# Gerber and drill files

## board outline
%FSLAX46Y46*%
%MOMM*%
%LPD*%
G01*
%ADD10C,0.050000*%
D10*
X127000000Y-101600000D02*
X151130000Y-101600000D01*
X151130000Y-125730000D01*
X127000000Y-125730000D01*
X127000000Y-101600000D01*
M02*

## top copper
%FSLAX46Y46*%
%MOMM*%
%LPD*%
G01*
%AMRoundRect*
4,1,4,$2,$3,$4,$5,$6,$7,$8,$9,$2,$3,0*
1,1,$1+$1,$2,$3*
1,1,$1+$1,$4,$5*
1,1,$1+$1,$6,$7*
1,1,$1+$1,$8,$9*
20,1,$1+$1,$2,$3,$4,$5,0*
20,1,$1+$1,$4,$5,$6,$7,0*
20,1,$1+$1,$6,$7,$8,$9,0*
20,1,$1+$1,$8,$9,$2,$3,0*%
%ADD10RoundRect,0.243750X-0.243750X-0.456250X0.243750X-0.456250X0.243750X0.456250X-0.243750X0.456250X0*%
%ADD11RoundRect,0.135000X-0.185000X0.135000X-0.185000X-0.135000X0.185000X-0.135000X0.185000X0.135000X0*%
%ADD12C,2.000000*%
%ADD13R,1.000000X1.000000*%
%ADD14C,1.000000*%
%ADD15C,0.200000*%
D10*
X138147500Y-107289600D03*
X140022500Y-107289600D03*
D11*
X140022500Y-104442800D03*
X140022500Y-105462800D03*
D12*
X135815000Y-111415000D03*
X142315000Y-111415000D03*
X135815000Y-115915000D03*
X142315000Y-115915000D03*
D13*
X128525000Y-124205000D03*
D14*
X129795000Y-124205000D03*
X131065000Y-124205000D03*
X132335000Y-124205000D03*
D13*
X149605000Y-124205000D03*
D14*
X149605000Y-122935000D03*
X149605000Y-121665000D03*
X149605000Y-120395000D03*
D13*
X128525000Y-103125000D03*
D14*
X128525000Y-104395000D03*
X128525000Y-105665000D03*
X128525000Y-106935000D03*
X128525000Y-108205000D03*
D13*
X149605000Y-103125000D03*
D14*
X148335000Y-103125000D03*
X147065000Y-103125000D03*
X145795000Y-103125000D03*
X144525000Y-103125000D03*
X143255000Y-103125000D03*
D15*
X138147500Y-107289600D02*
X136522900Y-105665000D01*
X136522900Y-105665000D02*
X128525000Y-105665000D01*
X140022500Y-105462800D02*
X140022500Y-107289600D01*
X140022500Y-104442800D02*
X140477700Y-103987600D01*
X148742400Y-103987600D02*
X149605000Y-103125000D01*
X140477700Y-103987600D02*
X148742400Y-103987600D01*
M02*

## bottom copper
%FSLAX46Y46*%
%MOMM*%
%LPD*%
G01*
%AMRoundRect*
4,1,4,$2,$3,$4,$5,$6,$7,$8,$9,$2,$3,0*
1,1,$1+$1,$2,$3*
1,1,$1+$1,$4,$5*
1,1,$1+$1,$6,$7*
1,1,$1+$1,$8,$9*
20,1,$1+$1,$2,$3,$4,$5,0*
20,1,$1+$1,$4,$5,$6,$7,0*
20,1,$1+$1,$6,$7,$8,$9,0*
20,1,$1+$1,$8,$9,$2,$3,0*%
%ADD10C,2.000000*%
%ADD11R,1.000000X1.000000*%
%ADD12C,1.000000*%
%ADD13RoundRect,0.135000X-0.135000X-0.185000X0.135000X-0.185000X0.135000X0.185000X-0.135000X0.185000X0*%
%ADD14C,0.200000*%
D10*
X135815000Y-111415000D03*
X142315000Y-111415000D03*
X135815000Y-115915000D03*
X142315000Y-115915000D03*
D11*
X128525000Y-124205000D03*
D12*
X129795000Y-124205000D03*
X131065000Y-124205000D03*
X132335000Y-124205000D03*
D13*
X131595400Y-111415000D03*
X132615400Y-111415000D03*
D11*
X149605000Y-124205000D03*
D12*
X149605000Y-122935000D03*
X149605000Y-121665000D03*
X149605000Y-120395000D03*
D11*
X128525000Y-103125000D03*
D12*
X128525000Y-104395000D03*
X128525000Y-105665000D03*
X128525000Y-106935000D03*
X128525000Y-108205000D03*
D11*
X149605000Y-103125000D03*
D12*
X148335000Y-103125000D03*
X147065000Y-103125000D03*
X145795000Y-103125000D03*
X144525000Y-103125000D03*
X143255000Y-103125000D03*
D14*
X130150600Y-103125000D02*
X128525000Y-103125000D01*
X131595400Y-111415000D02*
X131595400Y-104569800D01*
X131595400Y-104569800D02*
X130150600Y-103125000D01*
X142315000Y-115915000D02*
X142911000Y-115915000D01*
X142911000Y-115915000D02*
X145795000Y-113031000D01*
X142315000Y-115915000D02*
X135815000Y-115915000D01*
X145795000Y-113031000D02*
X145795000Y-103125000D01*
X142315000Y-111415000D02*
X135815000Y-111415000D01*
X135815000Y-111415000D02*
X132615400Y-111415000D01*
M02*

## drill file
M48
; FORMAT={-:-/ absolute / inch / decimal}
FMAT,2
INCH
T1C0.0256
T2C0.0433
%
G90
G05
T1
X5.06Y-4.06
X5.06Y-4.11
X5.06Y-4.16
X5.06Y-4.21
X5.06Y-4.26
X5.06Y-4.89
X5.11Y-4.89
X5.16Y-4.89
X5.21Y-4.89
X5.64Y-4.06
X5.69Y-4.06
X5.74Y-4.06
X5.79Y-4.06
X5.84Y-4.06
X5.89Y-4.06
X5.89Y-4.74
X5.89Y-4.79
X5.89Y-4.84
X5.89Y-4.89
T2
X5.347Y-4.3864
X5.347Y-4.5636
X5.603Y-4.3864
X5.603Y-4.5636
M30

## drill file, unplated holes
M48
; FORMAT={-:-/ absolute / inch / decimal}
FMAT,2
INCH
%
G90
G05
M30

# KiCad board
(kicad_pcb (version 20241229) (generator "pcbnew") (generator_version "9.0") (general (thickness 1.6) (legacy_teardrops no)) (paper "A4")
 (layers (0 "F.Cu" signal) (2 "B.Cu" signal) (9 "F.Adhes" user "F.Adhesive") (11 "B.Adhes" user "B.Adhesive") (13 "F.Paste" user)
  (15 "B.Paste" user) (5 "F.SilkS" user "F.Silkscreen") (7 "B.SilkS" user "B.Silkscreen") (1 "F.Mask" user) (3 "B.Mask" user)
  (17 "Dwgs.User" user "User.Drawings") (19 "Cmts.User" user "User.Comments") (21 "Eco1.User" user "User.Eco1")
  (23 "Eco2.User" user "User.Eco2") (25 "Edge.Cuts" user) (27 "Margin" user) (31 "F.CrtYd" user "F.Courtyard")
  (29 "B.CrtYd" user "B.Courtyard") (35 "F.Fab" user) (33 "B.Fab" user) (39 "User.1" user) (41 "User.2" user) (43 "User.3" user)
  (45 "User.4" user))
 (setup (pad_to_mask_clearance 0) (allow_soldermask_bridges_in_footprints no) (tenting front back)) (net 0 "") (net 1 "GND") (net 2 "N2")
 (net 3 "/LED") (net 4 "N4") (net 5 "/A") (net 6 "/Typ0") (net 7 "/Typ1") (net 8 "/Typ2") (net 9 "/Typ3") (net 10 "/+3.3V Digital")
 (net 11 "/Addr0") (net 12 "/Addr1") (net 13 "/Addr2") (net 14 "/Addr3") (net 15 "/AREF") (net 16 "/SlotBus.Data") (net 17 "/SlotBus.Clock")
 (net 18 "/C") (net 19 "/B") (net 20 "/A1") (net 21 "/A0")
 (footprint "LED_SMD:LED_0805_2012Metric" (layer "F.Cu") (at 139.085 107.2896)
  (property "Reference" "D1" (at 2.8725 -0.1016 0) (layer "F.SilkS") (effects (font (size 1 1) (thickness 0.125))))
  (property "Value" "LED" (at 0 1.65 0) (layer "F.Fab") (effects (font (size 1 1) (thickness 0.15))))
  (pad "1" smd roundrect (at -0.9375 0) (size 0.975 1.4) (layers "F.Cu" "F.Mask" "F.Paste") (roundrect_rratio 0.25) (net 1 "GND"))
  (pad "2" smd roundrect (at 0.9375 0) (size 0.975 1.4) (layers "F.Cu" "F.Mask" "F.Paste") (roundrect_rratio 0.25) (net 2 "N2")))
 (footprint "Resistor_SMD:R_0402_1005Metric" (layer "F.Cu") (at 140.0225 104.9528 -90)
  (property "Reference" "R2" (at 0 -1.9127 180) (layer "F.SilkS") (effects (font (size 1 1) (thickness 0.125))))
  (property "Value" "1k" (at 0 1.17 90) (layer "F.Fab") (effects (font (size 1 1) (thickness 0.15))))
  (pad "1" smd roundrect (at -0.51 0 270) (size 0.54 0.64) (layers "F.Cu" "F.Mask" "F.Paste") (roundrect_rratio 0.25) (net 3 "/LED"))
  (pad "2" smd roundrect (at 0.51 0 270) (size 0.54 0.64) (layers "F.Cu" "F.Mask" "F.Paste") (roundrect_rratio 0.25) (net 2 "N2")))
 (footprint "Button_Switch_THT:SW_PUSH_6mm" (layer "F.Cu") (at 135.815 111.415)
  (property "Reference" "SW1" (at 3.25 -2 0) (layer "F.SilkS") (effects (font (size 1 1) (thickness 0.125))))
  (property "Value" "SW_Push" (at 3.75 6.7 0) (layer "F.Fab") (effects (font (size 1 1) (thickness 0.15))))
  (pad "1" thru_hole circle (at 0 0 90) (size 2 2) (drill 1.1) (layers "*.Cu" "*.Mask") (remove_unused_layers no) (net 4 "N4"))
  (pad "1" thru_hole circle (at 6.5 0 90) (size 2 2) (drill 1.1) (layers "*.Cu" "*.Mask") (remove_unused_layers no) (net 4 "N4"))
  (pad "2" thru_hole circle (at 0 4.5 90) (size 2 2) (drill 1.1) (layers "*.Cu" "*.Mask") (remove_unused_layers no) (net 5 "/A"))
  (pad "2" thru_hole circle (at 6.5 4.5 90) (size 2 2) (drill 1.1) (layers "*.Cu" "*.Mask") (remove_unused_layers no) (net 5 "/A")))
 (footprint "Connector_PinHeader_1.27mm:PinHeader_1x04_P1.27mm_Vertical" (layer "B.Cu") (at 128.525 124.205 -90)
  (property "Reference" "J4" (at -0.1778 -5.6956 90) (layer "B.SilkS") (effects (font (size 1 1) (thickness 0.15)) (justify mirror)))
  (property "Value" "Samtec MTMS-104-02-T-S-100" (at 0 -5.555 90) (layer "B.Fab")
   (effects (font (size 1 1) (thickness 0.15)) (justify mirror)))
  (pad "1" thru_hole rect (at 0 0 270) (size 1 1) (drill 0.65) (layers "*.Cu" "*.Mask") (remove_unused_layers no) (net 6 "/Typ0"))
  (pad "2" thru_hole circle (at 0 -1.27 270) (size 1 1) (drill 0.65) (layers "*.Cu" "*.Mask") (remove_unused_layers no) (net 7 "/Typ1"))
  (pad "3" thru_hole circle (at 0 -2.54 270) (size 1 1) (drill 0.65) (layers "*.Cu" "*.Mask") (remove_unused_layers no) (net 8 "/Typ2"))
  (pad "4" thru_hole circle (at 0 -3.81 270) (size 1 1) (drill 0.65) (layers "*.Cu" "*.Mask") (remove_unused_layers no) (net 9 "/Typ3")))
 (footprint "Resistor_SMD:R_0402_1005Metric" (layer "B.Cu") (at 132.1054 111.415)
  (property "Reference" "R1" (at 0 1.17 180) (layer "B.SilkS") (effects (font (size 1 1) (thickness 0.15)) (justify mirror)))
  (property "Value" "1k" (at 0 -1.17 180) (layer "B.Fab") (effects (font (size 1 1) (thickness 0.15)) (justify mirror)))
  (pad "1" smd roundrect (at -0.51 0) (size 0.54 0.64) (layers "B.Cu" "B.Mask" "B.Paste") (roundrect_rratio 0.25) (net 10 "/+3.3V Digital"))
  (pad "2" smd roundrect (at 0.51 0) (size 0.54 0.64) (layers "B.Cu" "B.Mask" "B.Paste") (roundrect_rratio 0.25) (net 4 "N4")))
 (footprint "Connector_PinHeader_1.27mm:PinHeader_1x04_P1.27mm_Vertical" (layer "B.Cu") (at 149.605 124.205)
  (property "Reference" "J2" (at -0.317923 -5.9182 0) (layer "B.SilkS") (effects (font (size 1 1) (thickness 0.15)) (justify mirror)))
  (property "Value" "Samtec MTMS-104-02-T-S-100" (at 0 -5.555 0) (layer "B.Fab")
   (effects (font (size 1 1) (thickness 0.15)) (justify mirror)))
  (pad "1" thru_hole rect (at 0 0) (size 1 1) (drill 0.65) (layers "*.Cu" "*.Mask") (remove_unused_layers no) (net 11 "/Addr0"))
  (pad "2" thru_hole circle (at 0 -1.27) (size 1 1) (drill 0.65) (layers "*.Cu" "*.Mask") (remove_unused_layers no) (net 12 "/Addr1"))
  (pad "3" thru_hole circle (at 0 -2.54) (size 1 1) (drill 0.65) (layers "*.Cu" "*.Mask") (remove_unused_layers no) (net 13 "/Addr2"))
  (pad "4" thru_hole circle (at 0 -3.81) (size 1 1) (drill 0.65) (layers "*.Cu" "*.Mask") (remove_unused_layers no) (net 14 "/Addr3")))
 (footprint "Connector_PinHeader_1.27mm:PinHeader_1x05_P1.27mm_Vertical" (layer "B.Cu") (at 128.525 103.125 180)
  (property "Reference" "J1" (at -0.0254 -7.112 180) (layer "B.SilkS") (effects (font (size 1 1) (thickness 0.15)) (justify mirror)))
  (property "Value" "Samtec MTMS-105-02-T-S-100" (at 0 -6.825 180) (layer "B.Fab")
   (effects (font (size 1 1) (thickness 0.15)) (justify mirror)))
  (pad "1" thru_hole rect (at 0 0 180) (size 1 1) (drill 0.65) (layers "*.Cu" "*.Mask") (remove_unused_layers no) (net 10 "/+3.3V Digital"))
  (pad "2" thru_hole circle (at 0 -1.27 180) (size 1 1) (drill 0.65) (layers "*.Cu" "*.Mask") (remove_unused_layers no) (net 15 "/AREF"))
  (pad "3" thru_hole circle (at 0 -2.54 180) (size 1 1) (drill 0.65) (layers "*.Cu" "*.Mask") (remove_unused_layers no) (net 1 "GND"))
  (pad "4" thru_hole circle (at 0 -3.81 180) (size 1 1) (drill 0.65) (layers "*.Cu" "*.Mask") (remove_unused_layers no)
   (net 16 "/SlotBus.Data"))
  (pad "5" thru_hole circle (at 0 -5.08 180) (size 1 1) (drill 0.65) (layers "*.Cu" "*.Mask") (remove_unused_layers no)
   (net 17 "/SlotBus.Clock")))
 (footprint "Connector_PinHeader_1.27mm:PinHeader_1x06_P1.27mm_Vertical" (layer "B.Cu") (at 149.605 103.125 90)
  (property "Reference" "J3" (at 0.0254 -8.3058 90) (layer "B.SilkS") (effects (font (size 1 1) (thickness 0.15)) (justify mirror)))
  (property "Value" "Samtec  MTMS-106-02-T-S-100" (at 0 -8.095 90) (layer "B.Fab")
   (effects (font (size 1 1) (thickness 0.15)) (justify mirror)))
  (pad "1" thru_hole rect (at 0 0 90) (size 1 1) (drill 0.65) (layers "*.Cu" "*.Mask") (remove_unused_layers no) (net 3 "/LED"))
  (pad "2" thru_hole circle (at 0 -1.27 90) (size 1 1) (drill 0.65) (layers "*.Cu" "*.Mask") (remove_unused_layers no) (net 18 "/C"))
  (pad "3" thru_hole circle (at 0 -2.54 90) (size 1 1) (drill 0.65) (layers "*.Cu" "*.Mask") (remove_unused_layers no) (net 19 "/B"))
  (pad "4" thru_hole circle (at 0 -3.81 90) (size 1 1) (drill 0.65) (layers "*.Cu" "*.Mask") (remove_unused_layers no) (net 5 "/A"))
  (pad "5" thru_hole circle (at 0 -5.08 90) (size 1 1) (drill 0.65) (layers "*.Cu" "*.Mask") (remove_unused_layers no) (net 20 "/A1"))
  (pad "6" thru_hole circle (at 0 -6.35 90) (size 1 1) (drill 0.65) (layers "*.Cu" "*.Mask") (remove_unused_layers no) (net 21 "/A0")))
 (gr_rect (start 127 101.6) (end 151.13 125.73) (stroke (width 0.05) (type solid)) (fill no) (layer "Edge.Cuts"))
 (segment (start 138.1475 107.2896) (end 136.5229 105.665) (width 0.2) (layer "F.Cu") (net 1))
 (segment (start 136.5229 105.665) (end 128.525 105.665) (width 0.2) (layer "F.Cu") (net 1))
 (segment (start 140.0225 105.4628) (end 140.0225 107.2896) (width 0.2) (layer "F.Cu") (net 2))
 (segment (start 130.1506 103.125) (end 128.525 103.125) (width 0.2) (layer "B.Cu") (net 10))
 (segment (start 131.5954 111.415) (end 131.5954 104.5698) (width 0.2) (layer "B.Cu") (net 10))
 (segment (start 131.5954 104.5698) (end 130.1506 103.125) (width 0.2) (layer "B.Cu") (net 10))
 (segment (start 140.0225 104.4428) (end 140.4777 103.9876) (width 0.2) (layer "F.Cu") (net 3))
 (segment (start 148.7424 103.9876) (end 149.605 103.125) (width 0.2) (layer "F.Cu") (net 3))
 (segment (start 140.4777 103.9876) (end 148.7424 103.9876) (width 0.2) (layer "F.Cu") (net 3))
 (segment (start 142.315 115.915) (end 142.911 115.915) (width 0.2) (layer "B.Cu") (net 5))
 (segment (start 142.911 115.915) (end 145.795 113.031) (width 0.2) (layer "B.Cu") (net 5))
 (segment (start 142.315 115.915) (end 135.815 115.915) (width 0.2) (layer "B.Cu") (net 5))
 (segment (start 145.795 113.031) (end 145.795 103.125) (width 0.2) (layer "B.Cu") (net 5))
 (segment (start 142.315 111.415) (end 135.815 111.415) (width 0.2) (layer "B.Cu") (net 4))
 (segment (start 135.815 111.415) (end 132.6154 111.415) (width 0.2) (layer "B.Cu") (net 4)))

